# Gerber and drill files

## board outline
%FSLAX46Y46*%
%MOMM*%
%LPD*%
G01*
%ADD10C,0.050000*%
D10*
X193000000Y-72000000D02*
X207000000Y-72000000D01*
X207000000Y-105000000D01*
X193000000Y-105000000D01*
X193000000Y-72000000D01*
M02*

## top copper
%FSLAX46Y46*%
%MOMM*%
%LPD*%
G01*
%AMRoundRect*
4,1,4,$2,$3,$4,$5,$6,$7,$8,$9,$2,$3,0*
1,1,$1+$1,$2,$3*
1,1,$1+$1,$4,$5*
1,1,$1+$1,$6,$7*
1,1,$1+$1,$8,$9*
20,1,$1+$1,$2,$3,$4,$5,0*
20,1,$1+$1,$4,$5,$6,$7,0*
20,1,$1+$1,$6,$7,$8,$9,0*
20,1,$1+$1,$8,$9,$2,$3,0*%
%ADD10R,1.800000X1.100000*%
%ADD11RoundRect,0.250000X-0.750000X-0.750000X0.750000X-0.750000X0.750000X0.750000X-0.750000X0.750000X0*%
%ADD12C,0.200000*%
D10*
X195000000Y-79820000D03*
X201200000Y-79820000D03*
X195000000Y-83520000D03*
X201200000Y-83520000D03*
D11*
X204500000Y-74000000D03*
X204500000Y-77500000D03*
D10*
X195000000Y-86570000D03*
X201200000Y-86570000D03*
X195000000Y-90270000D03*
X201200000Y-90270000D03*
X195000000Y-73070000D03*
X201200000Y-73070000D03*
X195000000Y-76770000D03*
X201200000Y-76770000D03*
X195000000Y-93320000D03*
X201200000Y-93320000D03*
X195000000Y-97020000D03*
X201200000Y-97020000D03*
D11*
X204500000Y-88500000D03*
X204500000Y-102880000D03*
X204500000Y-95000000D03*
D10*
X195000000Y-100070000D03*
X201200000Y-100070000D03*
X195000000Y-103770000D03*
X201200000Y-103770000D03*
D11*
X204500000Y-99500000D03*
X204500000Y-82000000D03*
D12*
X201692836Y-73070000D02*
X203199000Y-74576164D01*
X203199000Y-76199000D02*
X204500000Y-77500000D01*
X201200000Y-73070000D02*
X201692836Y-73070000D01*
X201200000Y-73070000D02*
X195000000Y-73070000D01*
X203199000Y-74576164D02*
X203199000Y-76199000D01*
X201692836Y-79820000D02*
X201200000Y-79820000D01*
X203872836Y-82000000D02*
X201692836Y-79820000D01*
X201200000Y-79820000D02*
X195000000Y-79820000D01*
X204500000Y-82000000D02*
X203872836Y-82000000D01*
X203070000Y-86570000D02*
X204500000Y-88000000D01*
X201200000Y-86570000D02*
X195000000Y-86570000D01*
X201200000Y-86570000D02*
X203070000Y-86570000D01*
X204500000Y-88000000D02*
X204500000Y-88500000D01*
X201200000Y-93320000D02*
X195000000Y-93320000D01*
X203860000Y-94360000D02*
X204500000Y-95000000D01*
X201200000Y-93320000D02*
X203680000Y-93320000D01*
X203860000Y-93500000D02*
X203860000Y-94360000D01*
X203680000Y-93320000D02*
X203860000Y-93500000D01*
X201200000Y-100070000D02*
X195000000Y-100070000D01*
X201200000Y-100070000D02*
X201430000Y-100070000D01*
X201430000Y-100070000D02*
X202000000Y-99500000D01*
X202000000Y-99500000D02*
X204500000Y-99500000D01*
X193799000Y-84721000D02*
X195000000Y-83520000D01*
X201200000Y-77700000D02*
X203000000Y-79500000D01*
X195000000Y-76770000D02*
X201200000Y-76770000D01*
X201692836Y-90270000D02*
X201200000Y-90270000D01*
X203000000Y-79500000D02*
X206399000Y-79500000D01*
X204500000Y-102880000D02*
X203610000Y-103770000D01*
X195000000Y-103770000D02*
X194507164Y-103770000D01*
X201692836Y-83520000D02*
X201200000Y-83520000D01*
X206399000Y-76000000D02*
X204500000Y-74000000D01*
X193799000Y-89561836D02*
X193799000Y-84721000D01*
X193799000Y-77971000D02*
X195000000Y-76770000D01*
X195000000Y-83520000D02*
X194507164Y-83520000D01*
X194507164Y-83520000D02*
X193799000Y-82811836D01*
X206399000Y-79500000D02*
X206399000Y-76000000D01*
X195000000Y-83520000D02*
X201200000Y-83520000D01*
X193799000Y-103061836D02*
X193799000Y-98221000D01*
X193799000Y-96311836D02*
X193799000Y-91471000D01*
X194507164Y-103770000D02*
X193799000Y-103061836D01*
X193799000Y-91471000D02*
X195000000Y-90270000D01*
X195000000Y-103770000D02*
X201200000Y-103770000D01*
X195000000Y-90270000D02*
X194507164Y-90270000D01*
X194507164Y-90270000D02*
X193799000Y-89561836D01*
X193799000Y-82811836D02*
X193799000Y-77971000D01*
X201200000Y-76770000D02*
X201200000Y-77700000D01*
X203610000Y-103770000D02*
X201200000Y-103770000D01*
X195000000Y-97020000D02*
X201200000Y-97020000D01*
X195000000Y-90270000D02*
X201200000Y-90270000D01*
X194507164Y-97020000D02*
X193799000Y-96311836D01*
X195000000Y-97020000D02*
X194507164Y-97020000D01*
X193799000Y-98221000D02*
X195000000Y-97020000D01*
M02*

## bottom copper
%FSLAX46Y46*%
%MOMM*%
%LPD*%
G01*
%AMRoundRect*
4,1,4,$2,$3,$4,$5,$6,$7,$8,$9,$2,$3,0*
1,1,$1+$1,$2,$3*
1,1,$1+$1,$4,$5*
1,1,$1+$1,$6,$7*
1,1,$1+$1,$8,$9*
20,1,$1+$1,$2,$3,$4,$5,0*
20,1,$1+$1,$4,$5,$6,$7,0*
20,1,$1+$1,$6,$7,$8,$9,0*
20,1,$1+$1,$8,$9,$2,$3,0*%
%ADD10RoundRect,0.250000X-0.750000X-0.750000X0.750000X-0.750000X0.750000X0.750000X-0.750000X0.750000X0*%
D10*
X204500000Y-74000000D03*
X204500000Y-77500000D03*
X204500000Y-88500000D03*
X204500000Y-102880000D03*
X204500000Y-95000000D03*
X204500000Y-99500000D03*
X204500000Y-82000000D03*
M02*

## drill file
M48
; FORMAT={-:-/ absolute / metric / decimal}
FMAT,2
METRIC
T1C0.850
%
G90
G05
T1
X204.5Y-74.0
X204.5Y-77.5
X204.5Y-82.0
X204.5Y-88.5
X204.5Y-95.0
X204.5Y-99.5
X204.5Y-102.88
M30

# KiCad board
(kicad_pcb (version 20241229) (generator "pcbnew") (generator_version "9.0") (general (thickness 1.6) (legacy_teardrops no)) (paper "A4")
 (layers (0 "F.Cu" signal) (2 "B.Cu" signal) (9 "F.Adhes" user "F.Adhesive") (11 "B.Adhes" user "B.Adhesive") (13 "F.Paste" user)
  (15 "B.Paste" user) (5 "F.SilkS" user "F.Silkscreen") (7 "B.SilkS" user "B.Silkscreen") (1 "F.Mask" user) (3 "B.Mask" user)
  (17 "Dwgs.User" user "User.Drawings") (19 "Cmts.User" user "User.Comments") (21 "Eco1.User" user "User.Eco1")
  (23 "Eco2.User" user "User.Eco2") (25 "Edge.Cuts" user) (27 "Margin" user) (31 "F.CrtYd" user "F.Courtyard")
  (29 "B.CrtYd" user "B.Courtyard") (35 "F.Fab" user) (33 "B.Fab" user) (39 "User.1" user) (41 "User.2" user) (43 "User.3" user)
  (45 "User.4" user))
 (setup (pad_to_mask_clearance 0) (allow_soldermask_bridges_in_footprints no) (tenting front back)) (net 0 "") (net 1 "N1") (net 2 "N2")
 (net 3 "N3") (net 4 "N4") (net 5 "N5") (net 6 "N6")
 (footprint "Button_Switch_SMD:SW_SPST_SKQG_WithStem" (layer "F.Cu") (at 198.1 81.67)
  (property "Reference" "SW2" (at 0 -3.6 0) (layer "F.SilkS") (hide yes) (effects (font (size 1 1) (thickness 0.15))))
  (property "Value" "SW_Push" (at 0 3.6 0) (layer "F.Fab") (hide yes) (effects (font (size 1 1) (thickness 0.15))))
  (pad "1" smd rect (at -3.1 -1.85) (size 1.8 1.1) (layers "F.Cu" "F.Mask" "F.Paste") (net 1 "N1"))
  (pad "1" smd rect (at 3.1 -1.85) (size 1.8 1.1) (layers "F.Cu" "F.Mask" "F.Paste") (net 1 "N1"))
  (pad "2" smd rect (at -3.1 1.85) (size 1.8 1.1) (layers "F.Cu" "F.Mask" "F.Paste") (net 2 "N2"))
  (pad "2" smd rect (at 3.1 1.85) (size 1.8 1.1) (layers "F.Cu" "F.Mask" "F.Paste") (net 2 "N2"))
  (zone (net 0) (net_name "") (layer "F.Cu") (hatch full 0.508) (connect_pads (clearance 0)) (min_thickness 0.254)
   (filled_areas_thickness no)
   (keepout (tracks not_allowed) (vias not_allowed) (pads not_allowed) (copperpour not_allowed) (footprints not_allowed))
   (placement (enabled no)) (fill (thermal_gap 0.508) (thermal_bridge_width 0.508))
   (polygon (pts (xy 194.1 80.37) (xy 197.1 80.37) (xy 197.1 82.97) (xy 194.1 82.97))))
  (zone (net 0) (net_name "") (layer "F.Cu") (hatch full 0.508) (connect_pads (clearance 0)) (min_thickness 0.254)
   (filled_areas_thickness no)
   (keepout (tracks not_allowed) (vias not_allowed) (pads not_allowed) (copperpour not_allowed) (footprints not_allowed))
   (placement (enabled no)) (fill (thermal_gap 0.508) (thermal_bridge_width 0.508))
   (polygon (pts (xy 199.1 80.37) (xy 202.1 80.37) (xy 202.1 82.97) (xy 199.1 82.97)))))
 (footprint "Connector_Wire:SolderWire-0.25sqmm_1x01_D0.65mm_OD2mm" (layer "F.Cu") (at 204.5 74)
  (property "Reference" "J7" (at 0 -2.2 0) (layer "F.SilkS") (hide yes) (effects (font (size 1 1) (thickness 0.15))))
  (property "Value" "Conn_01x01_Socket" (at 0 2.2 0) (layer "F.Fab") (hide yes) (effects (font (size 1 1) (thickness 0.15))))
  (pad "1" thru_hole roundrect (at 0 0) (size 2 2) (drill 0.85) (layers "*.Cu" "*.Mask") (remove_unused_layers no) (roundrect_rratio 0.125)
   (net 2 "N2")))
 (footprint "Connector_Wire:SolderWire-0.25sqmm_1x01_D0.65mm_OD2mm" (layer "F.Cu") (at 204.5 77.5)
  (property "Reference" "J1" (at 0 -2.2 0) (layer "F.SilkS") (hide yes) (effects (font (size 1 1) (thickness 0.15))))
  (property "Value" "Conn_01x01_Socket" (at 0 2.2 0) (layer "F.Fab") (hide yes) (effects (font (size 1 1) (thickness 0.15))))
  (pad "1" thru_hole roundrect (at 0 0) (size 2 2) (drill 0.85) (layers "*.Cu" "*.Mask") (remove_unused_layers no) (roundrect_rratio 0.125)
   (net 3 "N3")))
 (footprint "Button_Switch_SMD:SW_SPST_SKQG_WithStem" (layer "F.Cu") (at 198.1 88.42)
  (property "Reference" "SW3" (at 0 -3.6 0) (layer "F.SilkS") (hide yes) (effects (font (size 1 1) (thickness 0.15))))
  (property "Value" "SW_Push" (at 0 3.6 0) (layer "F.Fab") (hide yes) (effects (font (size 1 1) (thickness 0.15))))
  (pad "1" smd rect (at -3.1 -1.85) (size 1.8 1.1) (layers "F.Cu" "F.Mask" "F.Paste") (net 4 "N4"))
  (pad "1" smd rect (at 3.1 -1.85) (size 1.8 1.1) (layers "F.Cu" "F.Mask" "F.Paste") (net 4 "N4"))
  (pad "2" smd rect (at -3.1 1.85) (size 1.8 1.1) (layers "F.Cu" "F.Mask" "F.Paste") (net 2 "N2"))
  (pad "2" smd rect (at 3.1 1.85) (size 1.8 1.1) (layers "F.Cu" "F.Mask" "F.Paste") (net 2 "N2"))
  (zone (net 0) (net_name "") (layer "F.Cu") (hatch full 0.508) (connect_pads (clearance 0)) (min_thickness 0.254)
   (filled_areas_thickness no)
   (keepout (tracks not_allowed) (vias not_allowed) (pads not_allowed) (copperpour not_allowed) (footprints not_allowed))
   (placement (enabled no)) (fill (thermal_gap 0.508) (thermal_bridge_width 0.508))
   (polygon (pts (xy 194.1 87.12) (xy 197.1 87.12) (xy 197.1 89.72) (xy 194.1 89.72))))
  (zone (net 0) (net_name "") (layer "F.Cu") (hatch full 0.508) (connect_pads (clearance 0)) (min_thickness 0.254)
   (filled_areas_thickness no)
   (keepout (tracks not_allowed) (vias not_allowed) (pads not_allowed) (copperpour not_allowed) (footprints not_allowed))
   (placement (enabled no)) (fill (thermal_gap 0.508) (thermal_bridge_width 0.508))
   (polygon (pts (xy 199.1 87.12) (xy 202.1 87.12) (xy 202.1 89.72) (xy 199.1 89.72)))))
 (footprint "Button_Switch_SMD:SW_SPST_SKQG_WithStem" (layer "F.Cu") (at 198.1 74.92)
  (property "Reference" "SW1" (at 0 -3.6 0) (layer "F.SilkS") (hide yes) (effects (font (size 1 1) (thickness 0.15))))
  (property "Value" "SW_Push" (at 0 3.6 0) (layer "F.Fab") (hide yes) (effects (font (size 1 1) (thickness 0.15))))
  (pad "1" smd rect (at -3.1 -1.85) (size 1.8 1.1) (layers "F.Cu" "F.Mask" "F.Paste") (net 3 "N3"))
  (pad "1" smd rect (at 3.1 -1.85) (size 1.8 1.1) (layers "F.Cu" "F.Mask" "F.Paste") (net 3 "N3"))
  (pad "2" smd rect (at -3.1 1.85) (size 1.8 1.1) (layers "F.Cu" "F.Mask" "F.Paste") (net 2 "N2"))
  (pad "2" smd rect (at 3.1 1.85) (size 1.8 1.1) (layers "F.Cu" "F.Mask" "F.Paste") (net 2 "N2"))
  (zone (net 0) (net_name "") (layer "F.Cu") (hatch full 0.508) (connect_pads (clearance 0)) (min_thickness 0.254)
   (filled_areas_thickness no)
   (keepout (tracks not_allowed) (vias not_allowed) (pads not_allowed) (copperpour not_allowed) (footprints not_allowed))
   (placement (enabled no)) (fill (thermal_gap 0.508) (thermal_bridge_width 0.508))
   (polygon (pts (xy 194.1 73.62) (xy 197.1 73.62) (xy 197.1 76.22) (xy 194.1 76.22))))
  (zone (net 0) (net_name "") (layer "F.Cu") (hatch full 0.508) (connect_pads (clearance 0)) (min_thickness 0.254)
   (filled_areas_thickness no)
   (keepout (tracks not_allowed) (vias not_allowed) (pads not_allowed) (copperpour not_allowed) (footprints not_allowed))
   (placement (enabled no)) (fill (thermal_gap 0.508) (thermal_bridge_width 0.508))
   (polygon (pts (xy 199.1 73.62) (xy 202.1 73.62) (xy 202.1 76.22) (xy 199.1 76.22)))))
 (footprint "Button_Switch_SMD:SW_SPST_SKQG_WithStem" (layer "F.Cu") (at 198.1 95.17)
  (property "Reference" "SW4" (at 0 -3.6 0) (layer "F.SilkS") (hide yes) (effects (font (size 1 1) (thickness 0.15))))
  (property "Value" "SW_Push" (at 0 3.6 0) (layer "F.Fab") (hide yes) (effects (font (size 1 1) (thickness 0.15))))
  (pad "1" smd rect (at -3.1 -1.85) (size 1.8 1.1) (layers "F.Cu" "F.Mask" "F.Paste") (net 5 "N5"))
  (pad "1" smd rect (at 3.1 -1.85) (size 1.8 1.1) (layers "F.Cu" "F.Mask" "F.Paste") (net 5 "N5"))
  (pad "2" smd rect (at -3.1 1.85) (size 1.8 1.1) (layers "F.Cu" "F.Mask" "F.Paste") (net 2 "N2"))
  (pad "2" smd rect (at 3.1 1.85) (size 1.8 1.1) (layers "F.Cu" "F.Mask" "F.Paste") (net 2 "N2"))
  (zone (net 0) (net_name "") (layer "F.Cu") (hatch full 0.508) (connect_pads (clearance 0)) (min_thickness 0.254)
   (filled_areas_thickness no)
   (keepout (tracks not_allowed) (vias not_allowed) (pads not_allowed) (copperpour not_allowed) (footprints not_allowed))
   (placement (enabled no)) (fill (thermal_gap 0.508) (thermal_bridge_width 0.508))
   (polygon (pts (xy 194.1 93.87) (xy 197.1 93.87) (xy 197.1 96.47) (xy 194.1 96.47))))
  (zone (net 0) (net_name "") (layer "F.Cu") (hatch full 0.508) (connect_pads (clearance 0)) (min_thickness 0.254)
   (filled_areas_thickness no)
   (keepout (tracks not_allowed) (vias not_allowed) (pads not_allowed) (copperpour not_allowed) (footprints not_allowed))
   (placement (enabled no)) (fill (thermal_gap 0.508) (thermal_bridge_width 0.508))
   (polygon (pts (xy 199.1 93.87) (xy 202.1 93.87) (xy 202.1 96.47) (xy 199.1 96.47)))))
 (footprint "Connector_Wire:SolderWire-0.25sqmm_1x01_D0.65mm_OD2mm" (layer "F.Cu") (at 204.5 88.5)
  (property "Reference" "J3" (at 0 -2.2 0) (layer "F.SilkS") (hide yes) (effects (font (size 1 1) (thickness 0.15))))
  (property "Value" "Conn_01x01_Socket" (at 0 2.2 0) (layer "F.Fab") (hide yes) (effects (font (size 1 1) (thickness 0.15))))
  (pad "1" thru_hole roundrect (at 0 0) (size 2 2) (drill 0.85) (layers "*.Cu" "*.Mask") (remove_unused_layers no) (roundrect_rratio 0.125)
   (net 4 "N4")))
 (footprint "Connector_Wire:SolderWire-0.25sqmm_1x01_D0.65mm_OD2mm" (layer "F.Cu") (at 204.5 102.88)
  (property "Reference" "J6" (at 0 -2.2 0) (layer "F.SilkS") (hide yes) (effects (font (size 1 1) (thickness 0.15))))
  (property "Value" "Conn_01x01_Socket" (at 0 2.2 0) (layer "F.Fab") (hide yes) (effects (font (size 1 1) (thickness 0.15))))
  (pad "1" thru_hole roundrect (at 0 0) (size 2 2) (drill 0.85) (layers "*.Cu" "*.Mask") (remove_unused_layers no) (roundrect_rratio 0.125)
   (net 2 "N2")))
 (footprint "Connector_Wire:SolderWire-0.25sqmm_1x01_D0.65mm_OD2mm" (layer "F.Cu") (at 204.5 95)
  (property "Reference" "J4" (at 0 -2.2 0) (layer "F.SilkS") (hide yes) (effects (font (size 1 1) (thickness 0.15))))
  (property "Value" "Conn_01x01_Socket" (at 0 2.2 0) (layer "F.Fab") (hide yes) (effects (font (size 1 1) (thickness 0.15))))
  (pad "1" thru_hole roundrect (at 0 0) (size 2 2) (drill 0.85) (layers "*.Cu" "*.Mask") (remove_unused_layers no) (roundrect_rratio 0.125)
   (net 5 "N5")))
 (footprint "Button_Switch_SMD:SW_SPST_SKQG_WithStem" (layer "F.Cu") (at 198.1 101.92)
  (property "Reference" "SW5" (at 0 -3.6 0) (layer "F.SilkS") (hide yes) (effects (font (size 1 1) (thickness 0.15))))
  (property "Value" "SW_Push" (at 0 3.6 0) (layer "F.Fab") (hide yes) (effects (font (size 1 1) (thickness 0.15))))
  (pad "1" smd rect (at -3.1 -1.85) (size 1.8 1.1) (layers "F.Cu" "F.Mask" "F.Paste") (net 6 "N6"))
  (pad "1" smd rect (at 3.1 -1.85) (size 1.8 1.1) (layers "F.Cu" "F.Mask" "F.Paste") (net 6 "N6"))
  (pad "2" smd rect (at -3.1 1.85) (size 1.8 1.1) (layers "F.Cu" "F.Mask" "F.Paste") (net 2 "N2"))
  (pad "2" smd rect (at 3.1 1.85) (size 1.8 1.1) (layers "F.Cu" "F.Mask" "F.Paste") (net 2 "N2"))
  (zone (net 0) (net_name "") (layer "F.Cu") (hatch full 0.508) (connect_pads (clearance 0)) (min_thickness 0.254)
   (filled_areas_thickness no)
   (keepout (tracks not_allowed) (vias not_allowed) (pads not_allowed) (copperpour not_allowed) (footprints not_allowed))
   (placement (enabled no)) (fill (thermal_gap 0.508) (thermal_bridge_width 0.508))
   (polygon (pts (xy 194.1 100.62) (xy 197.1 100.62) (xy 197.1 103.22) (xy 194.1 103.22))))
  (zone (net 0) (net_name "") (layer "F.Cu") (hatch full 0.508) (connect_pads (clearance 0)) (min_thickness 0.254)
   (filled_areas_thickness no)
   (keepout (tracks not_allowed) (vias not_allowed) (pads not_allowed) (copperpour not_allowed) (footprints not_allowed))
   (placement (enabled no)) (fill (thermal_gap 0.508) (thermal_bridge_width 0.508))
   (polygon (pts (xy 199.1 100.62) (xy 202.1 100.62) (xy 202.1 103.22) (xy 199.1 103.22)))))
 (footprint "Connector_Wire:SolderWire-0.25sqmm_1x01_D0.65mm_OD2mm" (layer "F.Cu") (at 204.5 99.5)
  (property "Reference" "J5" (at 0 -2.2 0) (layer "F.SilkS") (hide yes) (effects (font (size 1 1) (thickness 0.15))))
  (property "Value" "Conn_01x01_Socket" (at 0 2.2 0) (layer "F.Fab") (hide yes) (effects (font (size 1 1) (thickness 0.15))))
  (pad "1" thru_hole roundrect (at 0 0) (size 2 2) (drill 0.85) (layers "*.Cu" "*.Mask") (remove_unused_layers no) (roundrect_rratio 0.125)
   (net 6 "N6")))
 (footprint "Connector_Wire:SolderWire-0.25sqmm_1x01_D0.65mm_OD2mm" (layer "F.Cu") (at 204.5 82)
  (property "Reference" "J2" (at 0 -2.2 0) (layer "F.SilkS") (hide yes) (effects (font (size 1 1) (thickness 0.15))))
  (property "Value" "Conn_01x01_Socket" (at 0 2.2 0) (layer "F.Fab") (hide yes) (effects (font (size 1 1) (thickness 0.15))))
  (pad "1" thru_hole roundrect (at 0 0) (size 2 2) (drill 0.85) (layers "*.Cu" "*.Mask") (remove_unused_layers no) (roundrect_rratio 0.125)
   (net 1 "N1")))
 (gr_poly (pts (xy 193 72) (xy 207 72) (xy 207 105) (xy 193 105)) (stroke (width 0.05) (type solid)) (fill no) (layer "Edge.Cuts"))
 (segment (start 201.692836 73.07) (end 203.199 74.576164) (width 0.2) (layer "F.Cu") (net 3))
 (segment (start 203.199 76.199) (end 204.5 77.5) (width 0.2) (layer "F.Cu") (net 3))
 (segment (start 201.2 73.07) (end 201.692836 73.07) (width 0.2) (layer "F.Cu") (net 3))
 (segment (start 201.2 73.07) (end 195 73.07) (width 0.2) (layer "F.Cu") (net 3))
 (segment (start 203.199 74.576164) (end 203.199 76.199) (width 0.2) (layer "F.Cu") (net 3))
 (segment (start 201.692836 79.82) (end 201.2 79.82) (width 0.2) (layer "F.Cu") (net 1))
 (segment (start 203.872836 82) (end 201.692836 79.82) (width 0.2) (layer "F.Cu") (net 1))
 (segment (start 201.2 79.82) (end 195 79.82) (width 0.2) (layer "F.Cu") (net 1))
 (segment (start 204.5 82) (end 203.872836 82) (width 0.2) (layer "F.Cu") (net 1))
 (segment (start 203.07 86.57) (end 204.5 88) (width 0.2) (layer "F.Cu") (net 4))
 (segment (start 201.2 86.57) (end 195 86.57) (width 0.2) (layer "F.Cu") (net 4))
 (segment (start 201.2 86.57) (end 203.07 86.57) (width 0.2) (layer "F.Cu") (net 4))
 (segment (start 204.5 88) (end 204.5 88.5) (width 0.2) (layer "F.Cu") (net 4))
 (segment (start 201.2 93.32) (end 195 93.32) (width 0.2) (layer "F.Cu") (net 5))
 (segment (start 203.86 94.36) (end 204.5 95) (width 0.2) (layer "F.Cu") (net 5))
 (segment (start 201.2 93.32) (end 203.68 93.32) (width 0.2) (layer "F.Cu") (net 5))
 (segment (start 203.86 93.5) (end 203.86 94.36) (width 0.2) (layer "F.Cu") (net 5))
 (segment (start 203.68 93.32) (end 203.86 93.5) (width 0.2) (layer "F.Cu") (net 5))
 (segment (start 201.2 100.07) (end 195 100.07) (width 0.2) (layer "F.Cu") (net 6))
 (segment (start 201.2 100.07) (end 201.43 100.07) (width 0.2) (layer "F.Cu") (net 6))
 (segment (start 201.43 100.07) (end 202 99.5) (width 0.2) (layer "F.Cu") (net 6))
 (segment (start 202 99.5) (end 204.5 99.5) (width 0.2) (layer "F.Cu") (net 6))
 (segment (start 193.799 84.721) (end 195 83.52) (width 0.2) (layer "F.Cu") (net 2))
 (segment (start 201.2 77.7) (end 203 79.5) (width 0.2) (layer "F.Cu") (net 2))
 (segment (start 195 76.77) (end 201.2 76.77) (width 0.2) (layer "F.Cu") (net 2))
 (segment (start 201.692836 90.27) (end 201.2 90.27) (width 0.2) (layer "F.Cu") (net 2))
 (segment (start 203 79.5) (end 206.399 79.5) (width 0.2) (layer "F.Cu") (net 2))
 (segment (start 204.5 102.88) (end 203.61 103.77) (width 0.2) (layer "F.Cu") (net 2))
 (segment (start 195 103.77) (end 194.507164 103.77) (width 0.2) (layer "F.Cu") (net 2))
 (segment (start 201.692836 83.52) (end 201.2 83.52) (width 0.2) (layer "F.Cu") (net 2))
 (segment (start 206.399 76) (end 204.5 74) (width 0.2) (layer "F.Cu") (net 2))
 (segment (start 193.799 89.561836) (end 193.799 84.721) (width 0.2) (layer "F.Cu") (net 2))
 (segment (start 193.799 77.971) (end 195 76.77) (width 0.2) (layer "F.Cu") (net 2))
 (segment (start 195 83.52) (end 194.507164 83.52) (width 0.2) (layer "F.Cu") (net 2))
 (segment (start 194.507164 83.52) (end 193.799 82.811836) (width 0.2) (layer "F.Cu") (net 2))
 (segment (start 206.399 79.5) (end 206.399 76) (width 0.2) (layer "F.Cu") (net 2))
 (segment (start 195 83.52) (end 201.2 83.52) (width 0.2) (layer "F.Cu") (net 2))
 (segment (start 193.799 103.061836) (end 193.799 98.221) (width 0.2) (layer "F.Cu") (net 2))
 (segment (start 193.799 96.311836) (end 193.799 91.471) (width 0.2) (layer "F.Cu") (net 2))
 (segment (start 194.507164 103.77) (end 193.799 103.061836) (width 0.2) (layer "F.Cu") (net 2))
 (segment (start 193.799 91.471) (end 195 90.27) (width 0.2) (layer "F.Cu") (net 2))
 (segment (start 195 103.77) (end 201.2 103.77) (width 0.2) (layer "F.Cu") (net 2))
 (segment (start 195 90.27) (end 194.507164 90.27) (width 0.2) (layer "F.Cu") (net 2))
 (segment (start 194.507164 90.27) (end 193.799 89.561836) (width 0.2) (layer "F.Cu") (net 2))
 (segment (start 193.799 82.811836) (end 193.799 77.971) (width 0.2) (layer "F.Cu") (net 2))
 (segment (start 201.2 76.77) (end 201.2 77.7) (width 0.2) (layer "F.Cu") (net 2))
 (segment (start 203.61 103.77) (end 201.2 103.77) (width 0.2) (layer "F.Cu") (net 2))
 (segment (start 195 97.02) (end 201.2 97.02) (width 0.2) (layer "F.Cu") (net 2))
 (segment (start 195 90.27) (end 201.2 90.27) (width 0.2) (layer "F.Cu") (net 2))
 (segment (start 194.507164 97.02) (end 193.799 96.311836) (width 0.2) (layer "F.Cu") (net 2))
 (segment (start 195 97.02) (end 194.507164 97.02) (width 0.2) (layer "F.Cu") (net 2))
 (segment (start 193.799 98.221) (end 195 97.02) (width 0.2) (layer "F.Cu") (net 2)))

